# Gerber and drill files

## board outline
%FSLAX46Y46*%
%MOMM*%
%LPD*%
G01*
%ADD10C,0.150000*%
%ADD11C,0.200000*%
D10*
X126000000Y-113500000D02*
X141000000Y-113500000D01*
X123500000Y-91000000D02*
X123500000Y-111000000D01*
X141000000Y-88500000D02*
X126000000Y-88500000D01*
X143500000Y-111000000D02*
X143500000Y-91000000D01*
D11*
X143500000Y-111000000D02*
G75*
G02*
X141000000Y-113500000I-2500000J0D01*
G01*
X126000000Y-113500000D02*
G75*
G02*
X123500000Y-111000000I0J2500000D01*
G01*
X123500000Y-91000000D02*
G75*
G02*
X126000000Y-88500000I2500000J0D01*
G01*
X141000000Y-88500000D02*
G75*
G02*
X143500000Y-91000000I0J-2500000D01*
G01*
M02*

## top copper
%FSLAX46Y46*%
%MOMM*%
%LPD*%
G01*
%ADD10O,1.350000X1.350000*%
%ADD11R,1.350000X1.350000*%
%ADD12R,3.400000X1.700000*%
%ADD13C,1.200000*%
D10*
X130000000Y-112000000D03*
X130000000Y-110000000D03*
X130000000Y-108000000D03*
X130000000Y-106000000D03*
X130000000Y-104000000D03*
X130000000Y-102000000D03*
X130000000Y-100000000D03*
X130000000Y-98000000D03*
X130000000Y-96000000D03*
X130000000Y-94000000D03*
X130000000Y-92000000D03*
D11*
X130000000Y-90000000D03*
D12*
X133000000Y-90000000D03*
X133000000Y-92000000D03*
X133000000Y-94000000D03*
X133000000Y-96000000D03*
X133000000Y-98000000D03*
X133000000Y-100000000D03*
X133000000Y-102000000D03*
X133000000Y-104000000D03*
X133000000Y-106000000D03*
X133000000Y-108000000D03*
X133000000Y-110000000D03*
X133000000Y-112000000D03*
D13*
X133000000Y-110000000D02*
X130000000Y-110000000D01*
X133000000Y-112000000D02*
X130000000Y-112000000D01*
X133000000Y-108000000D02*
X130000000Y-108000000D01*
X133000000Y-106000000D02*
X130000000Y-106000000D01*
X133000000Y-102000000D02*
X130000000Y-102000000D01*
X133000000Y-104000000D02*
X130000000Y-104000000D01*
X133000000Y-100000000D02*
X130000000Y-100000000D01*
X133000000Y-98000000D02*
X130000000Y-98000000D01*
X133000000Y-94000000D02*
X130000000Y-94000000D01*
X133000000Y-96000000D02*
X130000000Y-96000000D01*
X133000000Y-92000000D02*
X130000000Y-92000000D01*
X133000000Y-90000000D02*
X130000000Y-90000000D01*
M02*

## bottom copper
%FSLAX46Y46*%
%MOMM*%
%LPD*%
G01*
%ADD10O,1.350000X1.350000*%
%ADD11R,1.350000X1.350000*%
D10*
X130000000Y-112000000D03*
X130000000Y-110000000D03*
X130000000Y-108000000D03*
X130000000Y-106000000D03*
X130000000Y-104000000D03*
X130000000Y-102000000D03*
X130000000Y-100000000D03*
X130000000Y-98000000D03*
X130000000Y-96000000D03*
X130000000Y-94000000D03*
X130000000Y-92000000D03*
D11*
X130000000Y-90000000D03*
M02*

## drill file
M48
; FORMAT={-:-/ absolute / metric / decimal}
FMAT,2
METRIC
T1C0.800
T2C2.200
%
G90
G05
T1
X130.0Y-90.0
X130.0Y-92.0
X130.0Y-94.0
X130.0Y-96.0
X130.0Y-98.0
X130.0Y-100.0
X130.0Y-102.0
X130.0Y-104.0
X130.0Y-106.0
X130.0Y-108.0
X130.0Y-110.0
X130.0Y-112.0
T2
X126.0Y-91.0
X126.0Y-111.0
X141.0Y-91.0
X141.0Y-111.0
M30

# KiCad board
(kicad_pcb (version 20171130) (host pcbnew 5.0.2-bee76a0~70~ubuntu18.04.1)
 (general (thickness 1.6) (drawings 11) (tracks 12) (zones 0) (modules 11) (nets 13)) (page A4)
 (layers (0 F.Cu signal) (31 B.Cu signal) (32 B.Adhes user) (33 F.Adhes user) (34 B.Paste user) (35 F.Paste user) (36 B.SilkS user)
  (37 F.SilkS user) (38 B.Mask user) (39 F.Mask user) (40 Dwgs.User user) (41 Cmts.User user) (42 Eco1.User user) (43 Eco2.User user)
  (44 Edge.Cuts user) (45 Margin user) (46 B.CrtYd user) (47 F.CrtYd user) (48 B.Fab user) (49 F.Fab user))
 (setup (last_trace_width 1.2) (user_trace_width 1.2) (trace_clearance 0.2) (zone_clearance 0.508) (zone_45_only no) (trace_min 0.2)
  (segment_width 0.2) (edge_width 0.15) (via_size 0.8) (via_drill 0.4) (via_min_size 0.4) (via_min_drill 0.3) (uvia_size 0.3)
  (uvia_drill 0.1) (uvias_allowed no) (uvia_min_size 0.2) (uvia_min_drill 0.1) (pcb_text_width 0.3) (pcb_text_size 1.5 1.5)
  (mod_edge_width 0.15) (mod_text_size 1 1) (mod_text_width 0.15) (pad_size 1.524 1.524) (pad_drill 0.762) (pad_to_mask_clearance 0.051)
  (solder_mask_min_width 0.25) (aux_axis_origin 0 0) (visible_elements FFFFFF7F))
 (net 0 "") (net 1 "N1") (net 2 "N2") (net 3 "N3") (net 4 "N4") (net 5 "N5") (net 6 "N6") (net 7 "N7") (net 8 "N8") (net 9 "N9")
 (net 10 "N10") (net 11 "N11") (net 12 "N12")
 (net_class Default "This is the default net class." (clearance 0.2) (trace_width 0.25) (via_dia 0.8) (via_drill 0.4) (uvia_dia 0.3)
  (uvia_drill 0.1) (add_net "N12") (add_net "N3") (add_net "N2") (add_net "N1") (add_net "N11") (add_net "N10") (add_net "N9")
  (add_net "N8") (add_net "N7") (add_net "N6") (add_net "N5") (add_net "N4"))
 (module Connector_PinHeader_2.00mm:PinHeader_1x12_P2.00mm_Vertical (layer F.Cu) (at 130 90)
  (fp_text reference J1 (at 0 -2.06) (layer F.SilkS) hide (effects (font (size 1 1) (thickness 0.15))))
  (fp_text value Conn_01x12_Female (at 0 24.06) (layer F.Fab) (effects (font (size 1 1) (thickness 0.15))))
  (pad 12 thru_hole oval (at 0 22) (size 1.35 1.35) (drill 0.8) (layers *.Cu *.Mask) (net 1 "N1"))
  (pad 11 thru_hole oval (at 0 20) (size 1.35 1.35) (drill 0.8) (layers *.Cu *.Mask) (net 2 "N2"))
  (pad 10 thru_hole oval (at 0 18) (size 1.35 1.35) (drill 0.8) (layers *.Cu *.Mask) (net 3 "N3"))
  (pad 9 thru_hole oval (at 0 16) (size 1.35 1.35) (drill 0.8) (layers *.Cu *.Mask) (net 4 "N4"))
  (pad 8 thru_hole oval (at 0 14) (size 1.35 1.35) (drill 0.8) (layers *.Cu *.Mask) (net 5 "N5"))
  (pad 7 thru_hole oval (at 0 12) (size 1.35 1.35) (drill 0.8) (layers *.Cu *.Mask) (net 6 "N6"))
  (pad 6 thru_hole oval (at 0 10) (size 1.35 1.35) (drill 0.8) (layers *.Cu *.Mask) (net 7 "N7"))
  (pad 5 thru_hole oval (at 0 8) (size 1.35 1.35) (drill 0.8) (layers *.Cu *.Mask) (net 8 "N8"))
  (pad 4 thru_hole oval (at 0 6) (size 1.35 1.35) (drill 0.8) (layers *.Cu *.Mask) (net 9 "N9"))
  (pad 3 thru_hole oval (at 0 4) (size 1.35 1.35) (drill 0.8) (layers *.Cu *.Mask) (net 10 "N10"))
  (pad 2 thru_hole oval (at 0 2) (size 1.35 1.35) (drill 0.8) (layers *.Cu *.Mask) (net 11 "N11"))
  (pad 1 thru_hole rect (at 0 0) (size 1.35 1.35) (drill 0.8) (layers *.Cu *.Mask) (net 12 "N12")))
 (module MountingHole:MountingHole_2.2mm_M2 (layer F.Cu) (at 141 111)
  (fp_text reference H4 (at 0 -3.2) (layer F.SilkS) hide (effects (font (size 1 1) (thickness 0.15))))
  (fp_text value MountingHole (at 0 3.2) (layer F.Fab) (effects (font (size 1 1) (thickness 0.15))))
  (pad 1 np_thru_hole circle (at 0 0) (size 2.2 2.2) (drill 2.2) (layers *.Cu *.Mask)))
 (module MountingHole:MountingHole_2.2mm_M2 (layer F.Cu) (at 141 91)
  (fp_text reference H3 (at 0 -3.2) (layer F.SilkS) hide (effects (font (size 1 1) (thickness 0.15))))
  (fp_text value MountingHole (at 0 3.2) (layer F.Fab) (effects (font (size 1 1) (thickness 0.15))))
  (pad 1 np_thru_hole circle (at 0 0) (size 2.2 2.2) (drill 2.2) (layers *.Cu *.Mask)))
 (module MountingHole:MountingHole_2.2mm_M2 (layer F.Cu) (at 126 111)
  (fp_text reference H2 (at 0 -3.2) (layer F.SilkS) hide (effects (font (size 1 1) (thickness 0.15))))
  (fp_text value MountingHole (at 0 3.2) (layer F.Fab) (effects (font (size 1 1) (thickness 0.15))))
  (pad 1 np_thru_hole circle (at 0 0) (size 2.2 2.2) (drill 2.2) (layers *.Cu *.Mask)))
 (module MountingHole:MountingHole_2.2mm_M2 (layer F.Cu) (at 126 91)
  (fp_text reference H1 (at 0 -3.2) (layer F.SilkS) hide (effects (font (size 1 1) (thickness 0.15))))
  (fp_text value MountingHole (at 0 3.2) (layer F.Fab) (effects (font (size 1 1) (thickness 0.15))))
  (pad 1 np_thru_hole circle (at 0 0) (size 2.2 2.2) (drill 2.2) (layers *.Cu *.Mask)))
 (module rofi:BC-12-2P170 (layer F.Cu) (at 135 91 180)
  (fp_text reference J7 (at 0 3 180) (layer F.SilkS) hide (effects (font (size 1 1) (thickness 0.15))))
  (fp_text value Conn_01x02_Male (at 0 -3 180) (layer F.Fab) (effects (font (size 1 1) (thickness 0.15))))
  (pad 2 smd rect (at 2 1 180) (size 3.4 1.7) (layers F.Cu F.Paste F.Mask) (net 12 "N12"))
  (pad 1 smd rect (at 2 -1 180) (size 3.4 1.7) (layers F.Cu F.Paste F.Mask) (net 11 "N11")))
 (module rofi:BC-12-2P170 (layer F.Cu) (at 135 95 180)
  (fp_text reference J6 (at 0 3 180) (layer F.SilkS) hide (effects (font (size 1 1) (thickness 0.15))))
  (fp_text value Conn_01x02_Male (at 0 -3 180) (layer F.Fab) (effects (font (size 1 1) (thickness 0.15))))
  (pad 2 smd rect (at 2 1 180) (size 3.4 1.7) (layers F.Cu F.Paste F.Mask) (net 10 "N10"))
  (pad 1 smd rect (at 2 -1 180) (size 3.4 1.7) (layers F.Cu F.Paste F.Mask) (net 9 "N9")))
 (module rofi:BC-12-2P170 (layer F.Cu) (at 135 99 180)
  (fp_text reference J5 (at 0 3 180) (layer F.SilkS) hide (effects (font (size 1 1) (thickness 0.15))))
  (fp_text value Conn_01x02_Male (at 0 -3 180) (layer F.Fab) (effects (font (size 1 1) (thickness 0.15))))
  (pad 2 smd rect (at 2 1 180) (size 3.4 1.7) (layers F.Cu F.Paste F.Mask) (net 8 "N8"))
  (pad 1 smd rect (at 2 -1 180) (size 3.4 1.7) (layers F.Cu F.Paste F.Mask) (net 7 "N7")))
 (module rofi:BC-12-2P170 (layer F.Cu) (at 135 103 180)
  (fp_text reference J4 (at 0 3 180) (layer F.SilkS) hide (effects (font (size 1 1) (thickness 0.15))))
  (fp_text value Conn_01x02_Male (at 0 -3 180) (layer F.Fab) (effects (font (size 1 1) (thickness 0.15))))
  (pad 2 smd rect (at 2 1 180) (size 3.4 1.7) (layers F.Cu F.Paste F.Mask) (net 6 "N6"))
  (pad 1 smd rect (at 2 -1 180) (size 3.4 1.7) (layers F.Cu F.Paste F.Mask) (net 5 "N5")))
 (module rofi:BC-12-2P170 (layer F.Cu) (at 135 107 180)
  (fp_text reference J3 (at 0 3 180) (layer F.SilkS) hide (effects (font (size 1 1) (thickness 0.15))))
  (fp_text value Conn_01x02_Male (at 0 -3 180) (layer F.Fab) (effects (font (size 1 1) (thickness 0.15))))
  (pad 2 smd rect (at 2 1 180) (size 3.4 1.7) (layers F.Cu F.Paste F.Mask) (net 4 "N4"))
  (pad 1 smd rect (at 2 -1 180) (size 3.4 1.7) (layers F.Cu F.Paste F.Mask) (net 3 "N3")))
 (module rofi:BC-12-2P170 (layer F.Cu) (at 135 111 180)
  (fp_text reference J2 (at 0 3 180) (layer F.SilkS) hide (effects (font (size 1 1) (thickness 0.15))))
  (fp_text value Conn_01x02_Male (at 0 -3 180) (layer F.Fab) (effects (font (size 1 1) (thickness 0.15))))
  (pad 2 smd rect (at 2 1 180) (size 3.4 1.7) (layers F.Cu F.Paste F.Mask) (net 2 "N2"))
  (pad 1 smd rect (at 2 -1 180) (size 3.4 1.7) (layers F.Cu F.Paste F.Mask) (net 1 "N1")))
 (gr_line (start 126 113.5) (end 141 113.5) (layer Edge.Cuts) (width 0.15))
 (gr_line (start 123.5 91) (end 123.5 111) (layer Edge.Cuts) (width 0.15))
 (gr_line (start 141 88.5) (end 126 88.5) (layer Edge.Cuts) (width 0.15))
 (gr_line (start 143.5 111) (end 143.5 91) (layer Edge.Cuts) (width 0.15))
 (gr_arc (start 141 111) (end 141 113.5) (angle -90) (layer Edge.Cuts) (width 0.2))
 (gr_arc (start 126 111) (end 123.5 111) (angle -90) (layer Edge.Cuts) (width 0.2))
 (gr_arc (start 126 91) (end 126 88.5) (angle -90) (layer Edge.Cuts) (width 0.2))
 (gr_arc (start 141 91) (end 143.5 91) (angle -90) (layer Edge.Cuts) (width 0.2))
 (segment (start 133 110) (end 130 110) (width 1.2) (layer F.Cu) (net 2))
 (segment (start 133 112) (end 130 112) (width 1.2) (layer F.Cu) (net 1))
 (segment (start 133 108) (end 130 108) (width 1.2) (layer F.Cu) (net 3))
 (segment (start 133 106) (end 130 106) (width 1.2) (layer F.Cu) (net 4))
 (segment (start 133 102) (end 130 102) (width 1.2) (layer F.Cu) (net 6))
 (segment (start 133 104) (end 130 104) (width 1.2) (layer F.Cu) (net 5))
 (segment (start 133 100) (end 130 100) (width 1.2) (layer F.Cu) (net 7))
 (segment (start 133 98) (end 130 98) (width 1.2) (layer F.Cu) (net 8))
 (segment (start 133 94) (end 130 94) (width 1.2) (layer F.Cu) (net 10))
 (segment (start 133 96) (end 130 96) (width 1.2) (layer F.Cu) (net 9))
 (segment (start 133 92) (end 130 92) (width 1.2) (layer F.Cu) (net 11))
 (segment (start 133 90) (end 130 90) (width 1.2) (layer F.Cu) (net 12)))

